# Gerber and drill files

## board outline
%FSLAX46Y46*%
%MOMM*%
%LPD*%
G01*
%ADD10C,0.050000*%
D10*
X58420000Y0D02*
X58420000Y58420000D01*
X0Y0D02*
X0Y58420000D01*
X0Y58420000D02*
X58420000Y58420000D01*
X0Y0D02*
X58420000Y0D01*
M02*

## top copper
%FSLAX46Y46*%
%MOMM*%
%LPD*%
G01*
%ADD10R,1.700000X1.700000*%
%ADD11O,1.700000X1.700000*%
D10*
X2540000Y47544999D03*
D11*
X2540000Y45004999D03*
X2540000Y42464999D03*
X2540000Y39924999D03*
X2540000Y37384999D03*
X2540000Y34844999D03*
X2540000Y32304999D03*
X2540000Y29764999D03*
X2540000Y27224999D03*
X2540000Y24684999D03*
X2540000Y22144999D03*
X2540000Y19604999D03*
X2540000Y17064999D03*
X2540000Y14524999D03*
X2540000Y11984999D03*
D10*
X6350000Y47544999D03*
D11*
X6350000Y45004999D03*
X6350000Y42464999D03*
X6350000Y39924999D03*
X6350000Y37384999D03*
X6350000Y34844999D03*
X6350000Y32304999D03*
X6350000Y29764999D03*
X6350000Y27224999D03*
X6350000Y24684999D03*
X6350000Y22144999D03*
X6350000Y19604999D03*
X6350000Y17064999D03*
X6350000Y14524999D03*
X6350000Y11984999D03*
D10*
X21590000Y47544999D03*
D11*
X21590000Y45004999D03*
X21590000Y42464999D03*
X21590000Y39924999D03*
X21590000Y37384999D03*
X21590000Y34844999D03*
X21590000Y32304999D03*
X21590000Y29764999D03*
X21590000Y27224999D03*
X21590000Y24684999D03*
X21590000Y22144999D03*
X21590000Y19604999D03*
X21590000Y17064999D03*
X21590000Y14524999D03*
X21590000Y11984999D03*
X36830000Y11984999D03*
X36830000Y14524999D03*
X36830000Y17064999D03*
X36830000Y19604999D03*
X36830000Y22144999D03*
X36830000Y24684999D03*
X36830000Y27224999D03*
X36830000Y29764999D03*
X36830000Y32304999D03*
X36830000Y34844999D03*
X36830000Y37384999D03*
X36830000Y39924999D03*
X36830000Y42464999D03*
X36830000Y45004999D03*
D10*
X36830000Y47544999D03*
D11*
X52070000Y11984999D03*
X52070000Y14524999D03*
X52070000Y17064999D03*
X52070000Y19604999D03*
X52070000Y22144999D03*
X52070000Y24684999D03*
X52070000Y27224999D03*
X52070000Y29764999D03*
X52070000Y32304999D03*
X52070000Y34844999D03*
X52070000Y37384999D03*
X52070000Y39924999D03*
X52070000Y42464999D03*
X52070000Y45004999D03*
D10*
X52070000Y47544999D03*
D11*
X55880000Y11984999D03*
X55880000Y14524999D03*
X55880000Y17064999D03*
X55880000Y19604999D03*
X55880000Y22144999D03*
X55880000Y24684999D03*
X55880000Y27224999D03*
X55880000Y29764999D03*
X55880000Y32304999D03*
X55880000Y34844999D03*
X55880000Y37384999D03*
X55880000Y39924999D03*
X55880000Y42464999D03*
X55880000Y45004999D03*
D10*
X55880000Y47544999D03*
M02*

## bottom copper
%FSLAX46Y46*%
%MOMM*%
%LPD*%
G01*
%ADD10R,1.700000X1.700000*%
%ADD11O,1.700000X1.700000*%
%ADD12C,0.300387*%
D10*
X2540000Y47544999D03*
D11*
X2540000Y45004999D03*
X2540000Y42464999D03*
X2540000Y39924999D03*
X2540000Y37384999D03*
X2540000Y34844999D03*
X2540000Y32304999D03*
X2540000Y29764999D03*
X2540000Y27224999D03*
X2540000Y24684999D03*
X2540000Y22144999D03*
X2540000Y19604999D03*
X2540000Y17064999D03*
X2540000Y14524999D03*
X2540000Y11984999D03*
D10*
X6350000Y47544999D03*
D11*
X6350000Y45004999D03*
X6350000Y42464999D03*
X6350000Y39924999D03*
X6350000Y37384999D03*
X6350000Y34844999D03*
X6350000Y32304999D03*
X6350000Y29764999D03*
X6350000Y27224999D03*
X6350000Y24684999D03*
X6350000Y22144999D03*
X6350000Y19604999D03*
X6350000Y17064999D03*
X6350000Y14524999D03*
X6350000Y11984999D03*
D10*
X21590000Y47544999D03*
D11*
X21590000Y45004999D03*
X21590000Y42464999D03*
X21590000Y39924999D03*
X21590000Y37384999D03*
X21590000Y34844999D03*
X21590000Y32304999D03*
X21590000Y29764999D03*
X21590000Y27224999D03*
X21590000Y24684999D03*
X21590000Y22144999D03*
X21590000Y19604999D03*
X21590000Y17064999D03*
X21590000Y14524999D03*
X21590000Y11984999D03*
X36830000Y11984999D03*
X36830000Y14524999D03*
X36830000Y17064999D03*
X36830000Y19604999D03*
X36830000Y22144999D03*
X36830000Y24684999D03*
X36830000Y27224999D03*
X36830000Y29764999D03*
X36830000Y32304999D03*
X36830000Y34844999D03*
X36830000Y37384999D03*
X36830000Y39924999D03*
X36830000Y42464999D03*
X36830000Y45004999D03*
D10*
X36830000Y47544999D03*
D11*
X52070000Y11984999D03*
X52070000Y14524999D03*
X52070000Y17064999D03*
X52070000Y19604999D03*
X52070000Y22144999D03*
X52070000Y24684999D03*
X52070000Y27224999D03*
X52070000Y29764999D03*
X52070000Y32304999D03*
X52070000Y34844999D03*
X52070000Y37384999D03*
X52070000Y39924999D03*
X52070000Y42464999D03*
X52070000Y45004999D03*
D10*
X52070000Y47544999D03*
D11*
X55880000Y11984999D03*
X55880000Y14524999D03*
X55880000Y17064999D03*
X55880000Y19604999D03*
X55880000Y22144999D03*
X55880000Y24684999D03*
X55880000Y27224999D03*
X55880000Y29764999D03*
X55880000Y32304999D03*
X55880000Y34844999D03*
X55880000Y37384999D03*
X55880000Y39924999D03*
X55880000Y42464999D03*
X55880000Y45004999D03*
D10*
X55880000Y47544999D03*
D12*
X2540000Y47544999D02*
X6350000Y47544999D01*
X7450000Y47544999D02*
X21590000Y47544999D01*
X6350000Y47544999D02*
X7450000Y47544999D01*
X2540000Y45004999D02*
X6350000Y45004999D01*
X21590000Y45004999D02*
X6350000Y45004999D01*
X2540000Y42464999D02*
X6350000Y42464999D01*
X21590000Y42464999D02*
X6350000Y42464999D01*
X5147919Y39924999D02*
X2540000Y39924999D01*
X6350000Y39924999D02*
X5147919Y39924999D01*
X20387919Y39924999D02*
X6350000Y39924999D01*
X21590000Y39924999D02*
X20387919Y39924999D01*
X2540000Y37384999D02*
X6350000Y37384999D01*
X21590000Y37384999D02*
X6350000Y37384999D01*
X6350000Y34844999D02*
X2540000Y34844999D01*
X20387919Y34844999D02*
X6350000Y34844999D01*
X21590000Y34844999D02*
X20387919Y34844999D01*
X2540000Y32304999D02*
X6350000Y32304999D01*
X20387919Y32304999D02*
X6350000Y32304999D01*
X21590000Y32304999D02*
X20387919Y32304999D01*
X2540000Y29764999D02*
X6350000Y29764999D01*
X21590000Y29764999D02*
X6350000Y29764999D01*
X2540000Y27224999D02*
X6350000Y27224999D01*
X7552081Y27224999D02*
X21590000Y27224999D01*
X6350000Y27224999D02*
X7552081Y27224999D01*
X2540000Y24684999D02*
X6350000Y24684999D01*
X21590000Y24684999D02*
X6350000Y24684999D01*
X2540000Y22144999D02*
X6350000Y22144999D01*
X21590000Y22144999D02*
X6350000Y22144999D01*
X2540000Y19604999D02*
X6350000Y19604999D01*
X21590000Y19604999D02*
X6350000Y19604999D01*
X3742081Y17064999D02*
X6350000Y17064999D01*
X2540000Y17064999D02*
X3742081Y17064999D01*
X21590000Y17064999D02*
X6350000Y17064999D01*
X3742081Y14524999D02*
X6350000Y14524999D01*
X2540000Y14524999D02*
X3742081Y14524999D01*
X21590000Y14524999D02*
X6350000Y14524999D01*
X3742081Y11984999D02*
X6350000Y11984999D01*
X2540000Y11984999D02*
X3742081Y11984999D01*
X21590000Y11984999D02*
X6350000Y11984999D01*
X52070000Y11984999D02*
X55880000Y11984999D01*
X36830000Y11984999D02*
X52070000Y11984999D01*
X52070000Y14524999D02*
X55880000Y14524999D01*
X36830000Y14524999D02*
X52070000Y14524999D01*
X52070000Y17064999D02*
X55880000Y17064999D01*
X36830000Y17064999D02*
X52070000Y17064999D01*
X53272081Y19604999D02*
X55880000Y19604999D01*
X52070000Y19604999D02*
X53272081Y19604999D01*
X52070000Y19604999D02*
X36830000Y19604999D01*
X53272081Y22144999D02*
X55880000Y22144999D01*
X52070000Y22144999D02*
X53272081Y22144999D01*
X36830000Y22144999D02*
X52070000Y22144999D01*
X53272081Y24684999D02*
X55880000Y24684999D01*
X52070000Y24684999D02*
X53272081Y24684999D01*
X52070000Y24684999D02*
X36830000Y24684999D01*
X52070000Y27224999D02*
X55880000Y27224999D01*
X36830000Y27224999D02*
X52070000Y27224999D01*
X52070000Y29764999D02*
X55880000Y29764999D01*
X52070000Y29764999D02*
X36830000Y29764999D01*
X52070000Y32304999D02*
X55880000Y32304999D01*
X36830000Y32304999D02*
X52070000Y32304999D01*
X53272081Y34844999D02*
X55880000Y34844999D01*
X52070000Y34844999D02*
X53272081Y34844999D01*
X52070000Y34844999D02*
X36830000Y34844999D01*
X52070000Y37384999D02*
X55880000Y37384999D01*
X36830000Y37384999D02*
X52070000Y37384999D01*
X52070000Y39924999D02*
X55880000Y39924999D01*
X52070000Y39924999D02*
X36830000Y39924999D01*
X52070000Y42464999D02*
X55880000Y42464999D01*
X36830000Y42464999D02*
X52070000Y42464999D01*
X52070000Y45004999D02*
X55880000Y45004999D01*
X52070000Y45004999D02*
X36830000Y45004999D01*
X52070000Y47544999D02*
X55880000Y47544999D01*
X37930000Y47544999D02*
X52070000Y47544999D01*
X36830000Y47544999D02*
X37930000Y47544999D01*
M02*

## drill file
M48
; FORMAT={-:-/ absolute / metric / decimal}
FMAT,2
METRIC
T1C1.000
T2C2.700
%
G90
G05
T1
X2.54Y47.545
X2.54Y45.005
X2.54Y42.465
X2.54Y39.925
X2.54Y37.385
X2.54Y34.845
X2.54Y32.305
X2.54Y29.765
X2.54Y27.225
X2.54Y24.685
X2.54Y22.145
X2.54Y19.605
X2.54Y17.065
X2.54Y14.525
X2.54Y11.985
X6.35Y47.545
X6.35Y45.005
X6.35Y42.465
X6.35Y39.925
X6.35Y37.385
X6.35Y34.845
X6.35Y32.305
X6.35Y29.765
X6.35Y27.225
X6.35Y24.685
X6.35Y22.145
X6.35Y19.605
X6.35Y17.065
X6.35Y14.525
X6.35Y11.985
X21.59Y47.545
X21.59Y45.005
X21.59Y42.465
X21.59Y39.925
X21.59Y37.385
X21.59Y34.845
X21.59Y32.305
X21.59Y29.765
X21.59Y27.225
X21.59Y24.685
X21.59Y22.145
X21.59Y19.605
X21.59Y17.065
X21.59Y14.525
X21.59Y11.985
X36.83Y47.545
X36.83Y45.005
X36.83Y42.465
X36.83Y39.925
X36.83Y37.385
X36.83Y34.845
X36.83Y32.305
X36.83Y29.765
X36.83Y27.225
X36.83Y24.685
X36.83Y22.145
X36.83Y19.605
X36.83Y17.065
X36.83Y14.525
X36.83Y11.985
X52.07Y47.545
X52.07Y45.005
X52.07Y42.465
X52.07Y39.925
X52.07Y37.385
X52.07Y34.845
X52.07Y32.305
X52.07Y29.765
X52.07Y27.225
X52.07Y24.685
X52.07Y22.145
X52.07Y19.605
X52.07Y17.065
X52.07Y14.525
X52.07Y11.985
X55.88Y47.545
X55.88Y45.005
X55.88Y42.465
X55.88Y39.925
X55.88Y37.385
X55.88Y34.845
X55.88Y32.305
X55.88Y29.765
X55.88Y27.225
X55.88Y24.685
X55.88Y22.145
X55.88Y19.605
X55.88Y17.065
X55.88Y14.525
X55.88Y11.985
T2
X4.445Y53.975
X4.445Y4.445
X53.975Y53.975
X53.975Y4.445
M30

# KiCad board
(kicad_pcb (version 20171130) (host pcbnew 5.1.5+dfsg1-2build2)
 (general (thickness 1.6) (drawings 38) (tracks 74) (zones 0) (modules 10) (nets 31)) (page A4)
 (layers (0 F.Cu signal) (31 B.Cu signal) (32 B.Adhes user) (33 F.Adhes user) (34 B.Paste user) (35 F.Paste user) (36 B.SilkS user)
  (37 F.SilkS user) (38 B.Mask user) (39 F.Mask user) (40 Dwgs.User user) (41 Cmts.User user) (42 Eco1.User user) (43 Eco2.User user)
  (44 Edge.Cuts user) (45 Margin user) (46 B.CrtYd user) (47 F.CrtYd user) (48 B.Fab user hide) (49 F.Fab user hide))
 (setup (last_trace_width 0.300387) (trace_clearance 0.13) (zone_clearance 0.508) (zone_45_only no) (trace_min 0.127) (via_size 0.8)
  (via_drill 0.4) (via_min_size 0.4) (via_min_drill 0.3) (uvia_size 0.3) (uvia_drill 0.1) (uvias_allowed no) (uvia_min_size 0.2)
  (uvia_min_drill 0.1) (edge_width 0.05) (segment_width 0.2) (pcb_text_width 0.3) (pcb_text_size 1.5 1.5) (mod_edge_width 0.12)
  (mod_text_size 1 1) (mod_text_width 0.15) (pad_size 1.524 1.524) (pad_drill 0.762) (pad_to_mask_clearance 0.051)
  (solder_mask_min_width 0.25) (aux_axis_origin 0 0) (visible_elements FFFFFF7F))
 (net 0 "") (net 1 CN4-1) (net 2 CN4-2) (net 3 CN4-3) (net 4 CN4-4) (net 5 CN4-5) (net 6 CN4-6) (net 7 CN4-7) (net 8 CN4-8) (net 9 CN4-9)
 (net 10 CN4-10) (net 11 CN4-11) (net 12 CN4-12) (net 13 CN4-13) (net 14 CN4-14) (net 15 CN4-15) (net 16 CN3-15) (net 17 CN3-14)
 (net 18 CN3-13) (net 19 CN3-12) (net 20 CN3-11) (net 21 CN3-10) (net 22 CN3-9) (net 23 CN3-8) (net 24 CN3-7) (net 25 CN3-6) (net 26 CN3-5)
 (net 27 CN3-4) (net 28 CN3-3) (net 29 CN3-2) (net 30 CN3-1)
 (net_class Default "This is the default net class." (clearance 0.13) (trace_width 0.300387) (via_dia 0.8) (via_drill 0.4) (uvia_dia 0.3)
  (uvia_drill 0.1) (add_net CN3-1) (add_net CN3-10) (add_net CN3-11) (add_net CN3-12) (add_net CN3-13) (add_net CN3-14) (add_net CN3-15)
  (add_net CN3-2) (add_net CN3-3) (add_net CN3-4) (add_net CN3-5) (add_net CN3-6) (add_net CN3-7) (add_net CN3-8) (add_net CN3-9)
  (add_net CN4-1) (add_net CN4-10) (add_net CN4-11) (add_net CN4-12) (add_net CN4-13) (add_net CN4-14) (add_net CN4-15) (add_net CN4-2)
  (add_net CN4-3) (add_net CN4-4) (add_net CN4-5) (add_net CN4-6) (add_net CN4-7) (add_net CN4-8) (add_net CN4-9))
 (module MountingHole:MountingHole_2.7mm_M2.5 (layer F.Cu) (at 53.975 -53.975)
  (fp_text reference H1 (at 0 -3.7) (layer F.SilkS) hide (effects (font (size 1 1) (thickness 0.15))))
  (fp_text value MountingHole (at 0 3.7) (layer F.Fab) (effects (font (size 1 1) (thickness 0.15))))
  (pad 1 np_thru_hole circle (at 0 0) (size 2.7 2.7) (drill 2.7) (layers *.Cu *.Mask)))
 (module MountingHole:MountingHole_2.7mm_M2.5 (layer F.Cu) (at 53.975 -4.445)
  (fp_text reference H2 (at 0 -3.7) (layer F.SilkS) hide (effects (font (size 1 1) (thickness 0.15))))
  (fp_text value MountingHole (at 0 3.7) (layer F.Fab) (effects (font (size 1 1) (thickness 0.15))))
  (pad 1 np_thru_hole circle (at 0 0) (size 2.7 2.7) (drill 2.7) (layers *.Cu *.Mask)))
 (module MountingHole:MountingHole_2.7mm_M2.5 (layer F.Cu) (at 4.445 -4.445)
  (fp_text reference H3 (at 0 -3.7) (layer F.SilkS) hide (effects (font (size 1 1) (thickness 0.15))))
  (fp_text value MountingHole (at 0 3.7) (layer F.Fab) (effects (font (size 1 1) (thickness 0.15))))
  (pad 1 np_thru_hole circle (at 0 0) (size 2.7 2.7) (drill 2.7) (layers *.Cu *.Mask)))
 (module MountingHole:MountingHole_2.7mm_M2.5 (layer F.Cu) (at 4.445 -53.975)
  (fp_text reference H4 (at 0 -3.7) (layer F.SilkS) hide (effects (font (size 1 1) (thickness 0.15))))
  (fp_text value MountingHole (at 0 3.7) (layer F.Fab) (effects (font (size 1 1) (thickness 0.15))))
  (pad 1 np_thru_hole circle (at 0 0) (size 2.7 2.7) (drill 2.7) (layers *.Cu *.Mask)))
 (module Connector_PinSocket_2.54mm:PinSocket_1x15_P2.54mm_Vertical (layer F.Cu) (at 2.54 -47.544999)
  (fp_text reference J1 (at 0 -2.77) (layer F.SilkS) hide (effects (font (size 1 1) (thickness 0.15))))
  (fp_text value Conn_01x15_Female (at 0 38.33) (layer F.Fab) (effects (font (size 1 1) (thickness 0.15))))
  (pad 1 thru_hole rect (at 0 0) (size 1.7 1.7) (drill 1) (layers *.Cu *.Mask) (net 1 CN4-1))
  (pad 2 thru_hole oval (at 0 2.54) (size 1.7 1.7) (drill 1) (layers *.Cu *.Mask) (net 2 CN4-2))
  (pad 3 thru_hole oval (at 0 5.08) (size 1.7 1.7) (drill 1) (layers *.Cu *.Mask) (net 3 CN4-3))
  (pad 4 thru_hole oval (at 0 7.62) (size 1.7 1.7) (drill 1) (layers *.Cu *.Mask) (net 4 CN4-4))
  (pad 5 thru_hole oval (at 0 10.16) (size 1.7 1.7) (drill 1) (layers *.Cu *.Mask) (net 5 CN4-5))
  (pad 6 thru_hole oval (at 0 12.7) (size 1.7 1.7) (drill 1) (layers *.Cu *.Mask) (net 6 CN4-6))
  (pad 7 thru_hole oval (at 0 15.24) (size 1.7 1.7) (drill 1) (layers *.Cu *.Mask) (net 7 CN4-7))
  (pad 8 thru_hole oval (at 0 17.78) (size 1.7 1.7) (drill 1) (layers *.Cu *.Mask) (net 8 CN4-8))
  (pad 9 thru_hole oval (at 0 20.32) (size 1.7 1.7) (drill 1) (layers *.Cu *.Mask) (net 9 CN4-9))
  (pad 10 thru_hole oval (at 0 22.86) (size 1.7 1.7) (drill 1) (layers *.Cu *.Mask) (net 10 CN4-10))
  (pad 11 thru_hole oval (at 0 25.4) (size 1.7 1.7) (drill 1) (layers *.Cu *.Mask) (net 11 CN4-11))
  (pad 12 thru_hole oval (at 0 27.94) (size 1.7 1.7) (drill 1) (layers *.Cu *.Mask) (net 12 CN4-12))
  (pad 13 thru_hole oval (at 0 30.48) (size 1.7 1.7) (drill 1) (layers *.Cu *.Mask) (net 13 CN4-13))
  (pad 14 thru_hole oval (at 0 33.02) (size 1.7 1.7) (drill 1) (layers *.Cu *.Mask) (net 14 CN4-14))
  (pad 15 thru_hole oval (at 0 35.56) (size 1.7 1.7) (drill 1) (layers *.Cu *.Mask) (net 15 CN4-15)))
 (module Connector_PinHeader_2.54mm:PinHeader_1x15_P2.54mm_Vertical (layer F.Cu) (at 6.35 -47.544999)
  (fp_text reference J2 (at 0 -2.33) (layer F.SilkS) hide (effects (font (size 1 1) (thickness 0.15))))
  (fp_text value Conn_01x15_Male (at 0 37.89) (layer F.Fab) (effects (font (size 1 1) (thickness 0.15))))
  (pad 1 thru_hole rect (at 0 0) (size 1.7 1.7) (drill 1) (layers *.Cu *.Mask) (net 1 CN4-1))
  (pad 2 thru_hole oval (at 0 2.54) (size 1.7 1.7) (drill 1) (layers *.Cu *.Mask) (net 2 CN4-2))
  (pad 3 thru_hole oval (at 0 5.08) (size 1.7 1.7) (drill 1) (layers *.Cu *.Mask) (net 3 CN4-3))
  (pad 4 thru_hole oval (at 0 7.62) (size 1.7 1.7) (drill 1) (layers *.Cu *.Mask) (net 4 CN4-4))
  (pad 5 thru_hole oval (at 0 10.16) (size 1.7 1.7) (drill 1) (layers *.Cu *.Mask) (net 5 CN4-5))
  (pad 6 thru_hole oval (at 0 12.7) (size 1.7 1.7) (drill 1) (layers *.Cu *.Mask) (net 6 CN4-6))
  (pad 7 thru_hole oval (at 0 15.24) (size 1.7 1.7) (drill 1) (layers *.Cu *.Mask) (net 7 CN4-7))
  (pad 8 thru_hole oval (at 0 17.78) (size 1.7 1.7) (drill 1) (layers *.Cu *.Mask) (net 8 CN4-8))
  (pad 9 thru_hole oval (at 0 20.32) (size 1.7 1.7) (drill 1) (layers *.Cu *.Mask) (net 9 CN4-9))
  (pad 10 thru_hole oval (at 0 22.86) (size 1.7 1.7) (drill 1) (layers *.Cu *.Mask) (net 10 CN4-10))
  (pad 11 thru_hole oval (at 0 25.4) (size 1.7 1.7) (drill 1) (layers *.Cu *.Mask) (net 11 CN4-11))
  (pad 12 thru_hole oval (at 0 27.94) (size 1.7 1.7) (drill 1) (layers *.Cu *.Mask) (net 12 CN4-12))
  (pad 13 thru_hole oval (at 0 30.48) (size 1.7 1.7) (drill 1) (layers *.Cu *.Mask) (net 13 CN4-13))
  (pad 14 thru_hole oval (at 0 33.02) (size 1.7 1.7) (drill 1) (layers *.Cu *.Mask) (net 14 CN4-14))
  (pad 15 thru_hole oval (at 0 35.56) (size 1.7 1.7) (drill 1) (layers *.Cu *.Mask) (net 15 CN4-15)))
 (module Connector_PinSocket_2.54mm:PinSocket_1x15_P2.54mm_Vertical (layer F.Cu) (at 21.59 -47.544999)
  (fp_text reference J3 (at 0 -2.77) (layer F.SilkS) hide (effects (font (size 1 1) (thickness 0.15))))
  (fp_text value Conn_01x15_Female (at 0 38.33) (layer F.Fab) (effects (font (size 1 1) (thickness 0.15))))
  (pad 1 thru_hole rect (at 0 0) (size 1.7 1.7) (drill 1) (layers *.Cu *.Mask) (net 1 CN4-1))
  (pad 2 thru_hole oval (at 0 2.54) (size 1.7 1.7) (drill 1) (layers *.Cu *.Mask) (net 2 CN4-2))
  (pad 3 thru_hole oval (at 0 5.08) (size 1.7 1.7) (drill 1) (layers *.Cu *.Mask) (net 3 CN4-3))
  (pad 4 thru_hole oval (at 0 7.62) (size 1.7 1.7) (drill 1) (layers *.Cu *.Mask) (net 4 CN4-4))
  (pad 5 thru_hole oval (at 0 10.16) (size 1.7 1.7) (drill 1) (layers *.Cu *.Mask) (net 5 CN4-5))
  (pad 6 thru_hole oval (at 0 12.7) (size 1.7 1.7) (drill 1) (layers *.Cu *.Mask) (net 6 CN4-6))
  (pad 7 thru_hole oval (at 0 15.24) (size 1.7 1.7) (drill 1) (layers *.Cu *.Mask) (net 7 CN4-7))
  (pad 8 thru_hole oval (at 0 17.78) (size 1.7 1.7) (drill 1) (layers *.Cu *.Mask) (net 8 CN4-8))
  (pad 9 thru_hole oval (at 0 20.32) (size 1.7 1.7) (drill 1) (layers *.Cu *.Mask) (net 9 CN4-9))
  (pad 10 thru_hole oval (at 0 22.86) (size 1.7 1.7) (drill 1) (layers *.Cu *.Mask) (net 10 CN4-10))
  (pad 11 thru_hole oval (at 0 25.4) (size 1.7 1.7) (drill 1) (layers *.Cu *.Mask) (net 11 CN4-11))
  (pad 12 thru_hole oval (at 0 27.94) (size 1.7 1.7) (drill 1) (layers *.Cu *.Mask) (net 12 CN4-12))
  (pad 13 thru_hole oval (at 0 30.48) (size 1.7 1.7) (drill 1) (layers *.Cu *.Mask) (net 13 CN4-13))
  (pad 14 thru_hole oval (at 0 33.02) (size 1.7 1.7) (drill 1) (layers *.Cu *.Mask) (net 14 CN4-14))
  (pad 15 thru_hole oval (at 0 35.56) (size 1.7 1.7) (drill 1) (layers *.Cu *.Mask) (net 15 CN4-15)))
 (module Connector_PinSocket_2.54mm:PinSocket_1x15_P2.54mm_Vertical (layer F.Cu) (at 36.83 -47.544999)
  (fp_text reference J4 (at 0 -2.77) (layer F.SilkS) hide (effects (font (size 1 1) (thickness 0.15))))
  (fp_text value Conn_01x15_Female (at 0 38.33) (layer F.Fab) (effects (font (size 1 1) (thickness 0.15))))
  (pad 15 thru_hole oval (at 0 35.56) (size 1.7 1.7) (drill 1) (layers *.Cu *.Mask) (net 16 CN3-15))
  (pad 14 thru_hole oval (at 0 33.02) (size 1.7 1.7) (drill 1) (layers *.Cu *.Mask) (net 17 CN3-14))
  (pad 13 thru_hole oval (at 0 30.48) (size 1.7 1.7) (drill 1) (layers *.Cu *.Mask) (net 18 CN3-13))
  (pad 12 thru_hole oval (at 0 27.94) (size 1.7 1.7) (drill 1) (layers *.Cu *.Mask) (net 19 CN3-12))
  (pad 11 thru_hole oval (at 0 25.4) (size 1.7 1.7) (drill 1) (layers *.Cu *.Mask) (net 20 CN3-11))
  (pad 10 thru_hole oval (at 0 22.86) (size 1.7 1.7) (drill 1) (layers *.Cu *.Mask) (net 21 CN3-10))
  (pad 9 thru_hole oval (at 0 20.32) (size 1.7 1.7) (drill 1) (layers *.Cu *.Mask) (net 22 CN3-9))
  (pad 8 thru_hole oval (at 0 17.78) (size 1.7 1.7) (drill 1) (layers *.Cu *.Mask) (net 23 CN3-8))
  (pad 7 thru_hole oval (at 0 15.24) (size 1.7 1.7) (drill 1) (layers *.Cu *.Mask) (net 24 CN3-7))
  (pad 6 thru_hole oval (at 0 12.7) (size 1.7 1.7) (drill 1) (layers *.Cu *.Mask) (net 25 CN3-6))
  (pad 5 thru_hole oval (at 0 10.16) (size 1.7 1.7) (drill 1) (layers *.Cu *.Mask) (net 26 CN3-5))
  (pad 4 thru_hole oval (at 0 7.62) (size 1.7 1.7) (drill 1) (layers *.Cu *.Mask) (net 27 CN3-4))
  (pad 3 thru_hole oval (at 0 5.08) (size 1.7 1.7) (drill 1) (layers *.Cu *.Mask) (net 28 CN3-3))
  (pad 2 thru_hole oval (at 0 2.54) (size 1.7 1.7) (drill 1) (layers *.Cu *.Mask) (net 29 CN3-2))
  (pad 1 thru_hole rect (at 0 0) (size 1.7 1.7) (drill 1) (layers *.Cu *.Mask) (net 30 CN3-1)))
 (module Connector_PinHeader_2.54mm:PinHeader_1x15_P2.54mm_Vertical (layer F.Cu) (at 52.07 -47.544999)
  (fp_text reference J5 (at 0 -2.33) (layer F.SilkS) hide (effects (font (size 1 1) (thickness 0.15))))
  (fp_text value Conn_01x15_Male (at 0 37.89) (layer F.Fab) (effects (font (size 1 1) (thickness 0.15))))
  (pad 15 thru_hole oval (at 0 35.56) (size 1.7 1.7) (drill 1) (layers *.Cu *.Mask) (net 16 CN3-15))
  (pad 14 thru_hole oval (at 0 33.02) (size 1.7 1.7) (drill 1) (layers *.Cu *.Mask) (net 17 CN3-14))
  (pad 13 thru_hole oval (at 0 30.48) (size 1.7 1.7) (drill 1) (layers *.Cu *.Mask) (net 18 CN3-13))
  (pad 12 thru_hole oval (at 0 27.94) (size 1.7 1.7) (drill 1) (layers *.Cu *.Mask) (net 19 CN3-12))
  (pad 11 thru_hole oval (at 0 25.4) (size 1.7 1.7) (drill 1) (layers *.Cu *.Mask) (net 20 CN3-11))
  (pad 10 thru_hole oval (at 0 22.86) (size 1.7 1.7) (drill 1) (layers *.Cu *.Mask) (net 21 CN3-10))
  (pad 9 thru_hole oval (at 0 20.32) (size 1.7 1.7) (drill 1) (layers *.Cu *.Mask) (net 22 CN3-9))
  (pad 8 thru_hole oval (at 0 17.78) (size 1.7 1.7) (drill 1) (layers *.Cu *.Mask) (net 23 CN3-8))
  (pad 7 thru_hole oval (at 0 15.24) (size 1.7 1.7) (drill 1) (layers *.Cu *.Mask) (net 24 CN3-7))
  (pad 6 thru_hole oval (at 0 12.7) (size 1.7 1.7) (drill 1) (layers *.Cu *.Mask) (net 25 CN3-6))
  (pad 5 thru_hole oval (at 0 10.16) (size 1.7 1.7) (drill 1) (layers *.Cu *.Mask) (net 26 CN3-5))
  (pad 4 thru_hole oval (at 0 7.62) (size 1.7 1.7) (drill 1) (layers *.Cu *.Mask) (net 27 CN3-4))
  (pad 3 thru_hole oval (at 0 5.08) (size 1.7 1.7) (drill 1) (layers *.Cu *.Mask) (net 28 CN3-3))
  (pad 2 thru_hole oval (at 0 2.54) (size 1.7 1.7) (drill 1) (layers *.Cu *.Mask) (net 29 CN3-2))
  (pad 1 thru_hole rect (at 0 0) (size 1.7 1.7) (drill 1) (layers *.Cu *.Mask) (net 30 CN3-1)))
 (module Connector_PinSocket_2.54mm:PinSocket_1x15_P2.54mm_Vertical (layer F.Cu) (at 55.88 -47.544999)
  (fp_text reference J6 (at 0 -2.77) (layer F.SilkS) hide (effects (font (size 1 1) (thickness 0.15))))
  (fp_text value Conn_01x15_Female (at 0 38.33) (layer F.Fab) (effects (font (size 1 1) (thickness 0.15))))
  (pad 15 thru_hole oval (at 0 35.56) (size 1.7 1.7) (drill 1) (layers *.Cu *.Mask) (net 16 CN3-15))
  (pad 14 thru_hole oval (at 0 33.02) (size 1.7 1.7) (drill 1) (layers *.Cu *.Mask) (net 17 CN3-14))
  (pad 13 thru_hole oval (at 0 30.48) (size 1.7 1.7) (drill 1) (layers *.Cu *.Mask) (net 18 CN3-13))
  (pad 12 thru_hole oval (at 0 27.94) (size 1.7 1.7) (drill 1) (layers *.Cu *.Mask) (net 19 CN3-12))
  (pad 11 thru_hole oval (at 0 25.4) (size 1.7 1.7) (drill 1) (layers *.Cu *.Mask) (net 20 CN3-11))
  (pad 10 thru_hole oval (at 0 22.86) (size 1.7 1.7) (drill 1) (layers *.Cu *.Mask) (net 21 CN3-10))
  (pad 9 thru_hole oval (at 0 20.32) (size 1.7 1.7) (drill 1) (layers *.Cu *.Mask) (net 22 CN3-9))
  (pad 8 thru_hole oval (at 0 17.78) (size 1.7 1.7) (drill 1) (layers *.Cu *.Mask) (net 23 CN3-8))
  (pad 7 thru_hole oval (at 0 15.24) (size 1.7 1.7) (drill 1) (layers *.Cu *.Mask) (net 24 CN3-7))
  (pad 6 thru_hole oval (at 0 12.7) (size 1.7 1.7) (drill 1) (layers *.Cu *.Mask) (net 25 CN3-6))
  (pad 5 thru_hole oval (at 0 10.16) (size 1.7 1.7) (drill 1) (layers *.Cu *.Mask) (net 26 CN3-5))
  (pad 4 thru_hole oval (at 0 7.62) (size 1.7 1.7) (drill 1) (layers *.Cu *.Mask) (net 27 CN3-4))
  (pad 3 thru_hole oval (at 0 5.08) (size 1.7 1.7) (drill 1) (layers *.Cu *.Mask) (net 28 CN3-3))
  (pad 2 thru_hole oval (at 0 2.54) (size 1.7 1.7) (drill 1) (layers *.Cu *.Mask) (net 29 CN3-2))
  (pad 1 thru_hole rect (at 0 0) (size 1.7 1.7) (drill 1) (layers *.Cu *.Mask) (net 30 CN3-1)))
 (gr_line (start 58.42 0) (end 58.42 -58.42) (layer Edge.Cuts) (width 0.05))
 (gr_line (start 0 0) (end 0 -58.42) (layer Edge.Cuts) (width 0.05))
 (gr_line (start 0 -58.42) (end 58.42 -58.42) (layer Edge.Cuts) (width 0.05))
 (gr_line (start 0 0) (end 58.42 0) (layer Edge.Cuts) (width 0.05))
 (segment (start 2.54 -47.544999) (end 6.35 -47.544999) (width 0.300387) (layer B.Cu) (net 1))
 (segment (start 7.45 -47.544999) (end 21.59 -47.544999) (width 0.300387) (layer B.Cu) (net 1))
 (segment (start 6.35 -47.544999) (end 7.45 -47.544999) (width 0.300387) (layer B.Cu) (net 1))
 (segment (start 2.54 -45.004999) (end 6.35 -45.004999) (width 0.300387) (layer B.Cu) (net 2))
 (segment (start 21.59 -45.004999) (end 6.35 -45.004999) (width 0.300387) (layer B.Cu) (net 2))
 (segment (start 2.54 -42.464999) (end 6.35 -42.464999) (width 0.300387) (layer B.Cu) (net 3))
 (segment (start 21.59 -42.464999) (end 6.35 -42.464999) (width 0.300387) (layer B.Cu) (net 3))
 (segment (start 5.147919 -39.924999) (end 2.54 -39.924999) (width 0.300387) (layer B.Cu) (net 4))
 (segment (start 6.35 -39.924999) (end 5.147919 -39.924999) (width 0.300387) (layer B.Cu) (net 4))
 (segment (start 20.387919 -39.924999) (end 6.35 -39.924999) (width 0.300387) (layer B.Cu) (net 4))
 (segment (start 21.59 -39.924999) (end 20.387919 -39.924999) (width 0.300387) (layer B.Cu) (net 4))
 (segment (start 2.54 -37.384999) (end 6.35 -37.384999) (width 0.300387) (layer B.Cu) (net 5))
 (segment (start 21.59 -37.384999) (end 6.35 -37.384999) (width 0.300387) (layer B.Cu) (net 5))
 (segment (start 6.35 -34.844999) (end 2.54 -34.844999) (width 0.300387) (layer B.Cu) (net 6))
 (segment (start 20.387919 -34.844999) (end 6.35 -34.844999) (width 0.300387) (layer B.Cu) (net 6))
 (segment (start 21.59 -34.844999) (end 20.387919 -34.844999) (width 0.300387) (layer B.Cu) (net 6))
 (segment (start 2.54 -32.304999) (end 6.35 -32.304999) (width 0.300387) (layer B.Cu) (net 7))
 (segment (start 20.387919 -32.304999) (end 6.35 -32.304999) (width 0.300387) (layer B.Cu) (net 7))
 (segment (start 21.59 -32.304999) (end 20.387919 -32.304999) (width 0.300387) (layer B.Cu) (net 7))
 (segment (start 2.54 -29.764999) (end 6.35 -29.764999) (width 0.300387) (layer B.Cu) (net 8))
 (segment (start 21.59 -29.764999) (end 6.35 -29.764999) (width 0.300387) (layer B.Cu) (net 8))
 (segment (start 2.54 -27.224999) (end 6.35 -27.224999) (width 0.300387) (layer B.Cu) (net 9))
 (segment (start 7.552081 -27.224999) (end 21.59 -27.224999) (width 0.300387) (layer B.Cu) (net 9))
 (segment (start 6.35 -27.224999) (end 7.552081 -27.224999) (width 0.300387) (layer B.Cu) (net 9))
 (segment (start 2.54 -24.684999) (end 6.35 -24.684999) (width 0.300387) (layer B.Cu) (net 10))
 (segment (start 21.59 -24.684999) (end 6.35 -24.684999) (width 0.300387) (layer B.Cu) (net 10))
 (segment (start 2.54 -22.144999) (end 6.35 -22.144999) (width 0.300387) (layer B.Cu) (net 11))
 (segment (start 21.59 -22.144999) (end 6.35 -22.144999) (width 0.300387) (layer B.Cu) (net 11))
 (segment (start 2.54 -19.604999) (end 6.35 -19.604999) (width 0.300387) (layer B.Cu) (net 12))
 (segment (start 21.59 -19.604999) (end 6.35 -19.604999) (width 0.300387) (layer B.Cu) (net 12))
 (segment (start 3.742081 -17.064999) (end 6.35 -17.064999) (width 0.300387) (layer B.Cu) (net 13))
 (segment (start 2.54 -17.064999) (end 3.742081 -17.064999) (width 0.300387) (layer B.Cu) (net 13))
 (segment (start 21.59 -17.064999) (end 6.35 -17.064999) (width 0.300387) (layer B.Cu) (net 13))
 (segment (start 3.742081 -14.524999) (end 6.35 -14.524999) (width 0.300387) (layer B.Cu) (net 14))
 (segment (start 2.54 -14.524999) (end 3.742081 -14.524999) (width 0.300387) (layer B.Cu) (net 14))
 (segment (start 21.59 -14.524999) (end 6.35 -14.524999) (width 0.300387) (layer B.Cu) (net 14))
 (segment (start 3.742081 -11.984999) (end 6.35 -11.984999) (width 0.300387) (layer B.Cu) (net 15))
 (segment (start 2.54 -11.984999) (end 3.742081 -11.984999) (width 0.300387) (layer B.Cu) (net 15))
 (segment (start 21.59 -11.984999) (end 6.35 -11.984999) (width 0.300387) (layer B.Cu) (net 15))
 (segment (start 52.07 -11.984999) (end 55.88 -11.984999) (width 0.300387) (layer B.Cu) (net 16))
 (segment (start 36.83 -11.984999) (end 52.07 -11.984999) (width 0.300387) (layer B.Cu) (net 16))
 (segment (start 52.07 -14.524999) (end 55.88 -14.524999) (width 0.300387) (layer B.Cu) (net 17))
 (segment (start 36.83 -14.524999) (end 52.07 -14.524999) (width 0.300387) (layer B.Cu) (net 17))
 (segment (start 52.07 -17.064999) (end 55.88 -17.064999) (width 0.300387) (layer B.Cu) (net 18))
 (segment (start 36.83 -17.064999) (end 52.07 -17.064999) (width 0.300387) (layer B.Cu) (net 18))
 (segment (start 53.272081 -19.604999) (end 55.88 -19.604999) (width 0.300387) (layer B.Cu) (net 19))
 (segment (start 52.07 -19.604999) (end 53.272081 -19.604999) (width 0.300387) (layer B.Cu) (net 19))
 (segment (start 52.07 -19.604999) (end 36.83 -19.604999) (width 0.300387) (layer B.Cu) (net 19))
 (segment (start 53.272081 -22.144999) (end 55.88 -22.144999) (width 0.300387) (layer B.Cu) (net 20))
 (segment (start 52.07 -22.144999) (end 53.272081 -22.144999) (width 0.300387) (layer B.Cu) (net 20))
 (segment (start 36.83 -22.144999) (end 52.07 -22.144999) (width 0.300387) (layer B.Cu) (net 20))
 (segment (start 53.272081 -24.684999) (end 55.88 -24.684999) (width 0.300387) (layer B.Cu) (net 21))
 (segment (start 52.07 -24.684999) (end 53.272081 -24.684999) (width 0.300387) (layer B.Cu) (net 21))
 (segment (start 52.07 -24.684999) (end 36.83 -24.684999) (width 0.300387) (layer B.Cu) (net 21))
 (segment (start 52.07 -27.224999) (end 55.88 -27.224999) (width 0.300387) (layer B.Cu) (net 22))
 (segment (start 36.83 -27.224999) (end 52.07 -27.224999) (width 0.300387) (layer B.Cu) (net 22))
 (segment (start 52.07 -29.764999) (end 55.88 -29.764999) (width 0.300387) (layer B.Cu) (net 23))
 (segment (start 52.07 -29.764999) (end 36.83 -29.764999) (width 0.300387) (layer B.Cu) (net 23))
 (segment (start 52.07 -32.304999) (end 55.88 -32.304999) (width 0.300387) (layer B.Cu) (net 24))
 (segment (start 36.83 -32.304999) (end 52.07 -32.304999) (width 0.300387) (layer B.Cu) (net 24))
 (segment (start 53.272081 -34.844999) (end 55.88 -34.844999) (width 0.300387) (layer B.Cu) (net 25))
 (segment (start 52.07 -34.844999) (end 53.272081 -34.844999) (width 0.300387) (layer B.Cu) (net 25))
 (segment (start 52.07 -34.844999) (end 36.83 -34.844999) (width 0.300387) (layer B.Cu) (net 25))
 (segment (start 52.07 -37.384999) (end 55.88 -37.384999) (width 0.300387) (layer B.Cu) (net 26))
 (segment (start 36.83 -37.384999) (end 52.07 -37.384999) (width 0.300387) (layer B.Cu) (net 26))
 (segment (start 52.07 -39.924999) (end 55.88 -39.924999) (width 0.300387) (layer B.Cu) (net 27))
 (segment (start 52.07 -39.924999) (end 36.83 -39.924999) (width 0.300387) (layer B.Cu) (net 27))
 (segment (start 52.07 -42.464999) (end 55.88 -42.464999) (width 0.300387) (layer B.Cu) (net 28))
 (segment (start 36.83 -42.464999) (end 52.07 -42.464999) (width 0.300387) (layer B.Cu) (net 28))
 (segment (start 52.07 -45.004999) (end 55.88 -45.004999) (width 0.300387) (layer B.Cu) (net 29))
 (segment (start 52.07 -45.004999) (end 36.83 -45.004999) (width 0.300387) (layer B.Cu) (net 29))
 (segment (start 52.07 -47.544999) (end 55.88 -47.544999) (width 0.300387) (layer B.Cu) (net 30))
 (segment (start 37.93 -47.544999) (end 52.07 -47.544999) (width 0.300387) (layer B.Cu) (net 30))
 (segment (start 36.83 -47.544999) (end 37.93 -47.544999) (width 0.300387) (layer B.Cu) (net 30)))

